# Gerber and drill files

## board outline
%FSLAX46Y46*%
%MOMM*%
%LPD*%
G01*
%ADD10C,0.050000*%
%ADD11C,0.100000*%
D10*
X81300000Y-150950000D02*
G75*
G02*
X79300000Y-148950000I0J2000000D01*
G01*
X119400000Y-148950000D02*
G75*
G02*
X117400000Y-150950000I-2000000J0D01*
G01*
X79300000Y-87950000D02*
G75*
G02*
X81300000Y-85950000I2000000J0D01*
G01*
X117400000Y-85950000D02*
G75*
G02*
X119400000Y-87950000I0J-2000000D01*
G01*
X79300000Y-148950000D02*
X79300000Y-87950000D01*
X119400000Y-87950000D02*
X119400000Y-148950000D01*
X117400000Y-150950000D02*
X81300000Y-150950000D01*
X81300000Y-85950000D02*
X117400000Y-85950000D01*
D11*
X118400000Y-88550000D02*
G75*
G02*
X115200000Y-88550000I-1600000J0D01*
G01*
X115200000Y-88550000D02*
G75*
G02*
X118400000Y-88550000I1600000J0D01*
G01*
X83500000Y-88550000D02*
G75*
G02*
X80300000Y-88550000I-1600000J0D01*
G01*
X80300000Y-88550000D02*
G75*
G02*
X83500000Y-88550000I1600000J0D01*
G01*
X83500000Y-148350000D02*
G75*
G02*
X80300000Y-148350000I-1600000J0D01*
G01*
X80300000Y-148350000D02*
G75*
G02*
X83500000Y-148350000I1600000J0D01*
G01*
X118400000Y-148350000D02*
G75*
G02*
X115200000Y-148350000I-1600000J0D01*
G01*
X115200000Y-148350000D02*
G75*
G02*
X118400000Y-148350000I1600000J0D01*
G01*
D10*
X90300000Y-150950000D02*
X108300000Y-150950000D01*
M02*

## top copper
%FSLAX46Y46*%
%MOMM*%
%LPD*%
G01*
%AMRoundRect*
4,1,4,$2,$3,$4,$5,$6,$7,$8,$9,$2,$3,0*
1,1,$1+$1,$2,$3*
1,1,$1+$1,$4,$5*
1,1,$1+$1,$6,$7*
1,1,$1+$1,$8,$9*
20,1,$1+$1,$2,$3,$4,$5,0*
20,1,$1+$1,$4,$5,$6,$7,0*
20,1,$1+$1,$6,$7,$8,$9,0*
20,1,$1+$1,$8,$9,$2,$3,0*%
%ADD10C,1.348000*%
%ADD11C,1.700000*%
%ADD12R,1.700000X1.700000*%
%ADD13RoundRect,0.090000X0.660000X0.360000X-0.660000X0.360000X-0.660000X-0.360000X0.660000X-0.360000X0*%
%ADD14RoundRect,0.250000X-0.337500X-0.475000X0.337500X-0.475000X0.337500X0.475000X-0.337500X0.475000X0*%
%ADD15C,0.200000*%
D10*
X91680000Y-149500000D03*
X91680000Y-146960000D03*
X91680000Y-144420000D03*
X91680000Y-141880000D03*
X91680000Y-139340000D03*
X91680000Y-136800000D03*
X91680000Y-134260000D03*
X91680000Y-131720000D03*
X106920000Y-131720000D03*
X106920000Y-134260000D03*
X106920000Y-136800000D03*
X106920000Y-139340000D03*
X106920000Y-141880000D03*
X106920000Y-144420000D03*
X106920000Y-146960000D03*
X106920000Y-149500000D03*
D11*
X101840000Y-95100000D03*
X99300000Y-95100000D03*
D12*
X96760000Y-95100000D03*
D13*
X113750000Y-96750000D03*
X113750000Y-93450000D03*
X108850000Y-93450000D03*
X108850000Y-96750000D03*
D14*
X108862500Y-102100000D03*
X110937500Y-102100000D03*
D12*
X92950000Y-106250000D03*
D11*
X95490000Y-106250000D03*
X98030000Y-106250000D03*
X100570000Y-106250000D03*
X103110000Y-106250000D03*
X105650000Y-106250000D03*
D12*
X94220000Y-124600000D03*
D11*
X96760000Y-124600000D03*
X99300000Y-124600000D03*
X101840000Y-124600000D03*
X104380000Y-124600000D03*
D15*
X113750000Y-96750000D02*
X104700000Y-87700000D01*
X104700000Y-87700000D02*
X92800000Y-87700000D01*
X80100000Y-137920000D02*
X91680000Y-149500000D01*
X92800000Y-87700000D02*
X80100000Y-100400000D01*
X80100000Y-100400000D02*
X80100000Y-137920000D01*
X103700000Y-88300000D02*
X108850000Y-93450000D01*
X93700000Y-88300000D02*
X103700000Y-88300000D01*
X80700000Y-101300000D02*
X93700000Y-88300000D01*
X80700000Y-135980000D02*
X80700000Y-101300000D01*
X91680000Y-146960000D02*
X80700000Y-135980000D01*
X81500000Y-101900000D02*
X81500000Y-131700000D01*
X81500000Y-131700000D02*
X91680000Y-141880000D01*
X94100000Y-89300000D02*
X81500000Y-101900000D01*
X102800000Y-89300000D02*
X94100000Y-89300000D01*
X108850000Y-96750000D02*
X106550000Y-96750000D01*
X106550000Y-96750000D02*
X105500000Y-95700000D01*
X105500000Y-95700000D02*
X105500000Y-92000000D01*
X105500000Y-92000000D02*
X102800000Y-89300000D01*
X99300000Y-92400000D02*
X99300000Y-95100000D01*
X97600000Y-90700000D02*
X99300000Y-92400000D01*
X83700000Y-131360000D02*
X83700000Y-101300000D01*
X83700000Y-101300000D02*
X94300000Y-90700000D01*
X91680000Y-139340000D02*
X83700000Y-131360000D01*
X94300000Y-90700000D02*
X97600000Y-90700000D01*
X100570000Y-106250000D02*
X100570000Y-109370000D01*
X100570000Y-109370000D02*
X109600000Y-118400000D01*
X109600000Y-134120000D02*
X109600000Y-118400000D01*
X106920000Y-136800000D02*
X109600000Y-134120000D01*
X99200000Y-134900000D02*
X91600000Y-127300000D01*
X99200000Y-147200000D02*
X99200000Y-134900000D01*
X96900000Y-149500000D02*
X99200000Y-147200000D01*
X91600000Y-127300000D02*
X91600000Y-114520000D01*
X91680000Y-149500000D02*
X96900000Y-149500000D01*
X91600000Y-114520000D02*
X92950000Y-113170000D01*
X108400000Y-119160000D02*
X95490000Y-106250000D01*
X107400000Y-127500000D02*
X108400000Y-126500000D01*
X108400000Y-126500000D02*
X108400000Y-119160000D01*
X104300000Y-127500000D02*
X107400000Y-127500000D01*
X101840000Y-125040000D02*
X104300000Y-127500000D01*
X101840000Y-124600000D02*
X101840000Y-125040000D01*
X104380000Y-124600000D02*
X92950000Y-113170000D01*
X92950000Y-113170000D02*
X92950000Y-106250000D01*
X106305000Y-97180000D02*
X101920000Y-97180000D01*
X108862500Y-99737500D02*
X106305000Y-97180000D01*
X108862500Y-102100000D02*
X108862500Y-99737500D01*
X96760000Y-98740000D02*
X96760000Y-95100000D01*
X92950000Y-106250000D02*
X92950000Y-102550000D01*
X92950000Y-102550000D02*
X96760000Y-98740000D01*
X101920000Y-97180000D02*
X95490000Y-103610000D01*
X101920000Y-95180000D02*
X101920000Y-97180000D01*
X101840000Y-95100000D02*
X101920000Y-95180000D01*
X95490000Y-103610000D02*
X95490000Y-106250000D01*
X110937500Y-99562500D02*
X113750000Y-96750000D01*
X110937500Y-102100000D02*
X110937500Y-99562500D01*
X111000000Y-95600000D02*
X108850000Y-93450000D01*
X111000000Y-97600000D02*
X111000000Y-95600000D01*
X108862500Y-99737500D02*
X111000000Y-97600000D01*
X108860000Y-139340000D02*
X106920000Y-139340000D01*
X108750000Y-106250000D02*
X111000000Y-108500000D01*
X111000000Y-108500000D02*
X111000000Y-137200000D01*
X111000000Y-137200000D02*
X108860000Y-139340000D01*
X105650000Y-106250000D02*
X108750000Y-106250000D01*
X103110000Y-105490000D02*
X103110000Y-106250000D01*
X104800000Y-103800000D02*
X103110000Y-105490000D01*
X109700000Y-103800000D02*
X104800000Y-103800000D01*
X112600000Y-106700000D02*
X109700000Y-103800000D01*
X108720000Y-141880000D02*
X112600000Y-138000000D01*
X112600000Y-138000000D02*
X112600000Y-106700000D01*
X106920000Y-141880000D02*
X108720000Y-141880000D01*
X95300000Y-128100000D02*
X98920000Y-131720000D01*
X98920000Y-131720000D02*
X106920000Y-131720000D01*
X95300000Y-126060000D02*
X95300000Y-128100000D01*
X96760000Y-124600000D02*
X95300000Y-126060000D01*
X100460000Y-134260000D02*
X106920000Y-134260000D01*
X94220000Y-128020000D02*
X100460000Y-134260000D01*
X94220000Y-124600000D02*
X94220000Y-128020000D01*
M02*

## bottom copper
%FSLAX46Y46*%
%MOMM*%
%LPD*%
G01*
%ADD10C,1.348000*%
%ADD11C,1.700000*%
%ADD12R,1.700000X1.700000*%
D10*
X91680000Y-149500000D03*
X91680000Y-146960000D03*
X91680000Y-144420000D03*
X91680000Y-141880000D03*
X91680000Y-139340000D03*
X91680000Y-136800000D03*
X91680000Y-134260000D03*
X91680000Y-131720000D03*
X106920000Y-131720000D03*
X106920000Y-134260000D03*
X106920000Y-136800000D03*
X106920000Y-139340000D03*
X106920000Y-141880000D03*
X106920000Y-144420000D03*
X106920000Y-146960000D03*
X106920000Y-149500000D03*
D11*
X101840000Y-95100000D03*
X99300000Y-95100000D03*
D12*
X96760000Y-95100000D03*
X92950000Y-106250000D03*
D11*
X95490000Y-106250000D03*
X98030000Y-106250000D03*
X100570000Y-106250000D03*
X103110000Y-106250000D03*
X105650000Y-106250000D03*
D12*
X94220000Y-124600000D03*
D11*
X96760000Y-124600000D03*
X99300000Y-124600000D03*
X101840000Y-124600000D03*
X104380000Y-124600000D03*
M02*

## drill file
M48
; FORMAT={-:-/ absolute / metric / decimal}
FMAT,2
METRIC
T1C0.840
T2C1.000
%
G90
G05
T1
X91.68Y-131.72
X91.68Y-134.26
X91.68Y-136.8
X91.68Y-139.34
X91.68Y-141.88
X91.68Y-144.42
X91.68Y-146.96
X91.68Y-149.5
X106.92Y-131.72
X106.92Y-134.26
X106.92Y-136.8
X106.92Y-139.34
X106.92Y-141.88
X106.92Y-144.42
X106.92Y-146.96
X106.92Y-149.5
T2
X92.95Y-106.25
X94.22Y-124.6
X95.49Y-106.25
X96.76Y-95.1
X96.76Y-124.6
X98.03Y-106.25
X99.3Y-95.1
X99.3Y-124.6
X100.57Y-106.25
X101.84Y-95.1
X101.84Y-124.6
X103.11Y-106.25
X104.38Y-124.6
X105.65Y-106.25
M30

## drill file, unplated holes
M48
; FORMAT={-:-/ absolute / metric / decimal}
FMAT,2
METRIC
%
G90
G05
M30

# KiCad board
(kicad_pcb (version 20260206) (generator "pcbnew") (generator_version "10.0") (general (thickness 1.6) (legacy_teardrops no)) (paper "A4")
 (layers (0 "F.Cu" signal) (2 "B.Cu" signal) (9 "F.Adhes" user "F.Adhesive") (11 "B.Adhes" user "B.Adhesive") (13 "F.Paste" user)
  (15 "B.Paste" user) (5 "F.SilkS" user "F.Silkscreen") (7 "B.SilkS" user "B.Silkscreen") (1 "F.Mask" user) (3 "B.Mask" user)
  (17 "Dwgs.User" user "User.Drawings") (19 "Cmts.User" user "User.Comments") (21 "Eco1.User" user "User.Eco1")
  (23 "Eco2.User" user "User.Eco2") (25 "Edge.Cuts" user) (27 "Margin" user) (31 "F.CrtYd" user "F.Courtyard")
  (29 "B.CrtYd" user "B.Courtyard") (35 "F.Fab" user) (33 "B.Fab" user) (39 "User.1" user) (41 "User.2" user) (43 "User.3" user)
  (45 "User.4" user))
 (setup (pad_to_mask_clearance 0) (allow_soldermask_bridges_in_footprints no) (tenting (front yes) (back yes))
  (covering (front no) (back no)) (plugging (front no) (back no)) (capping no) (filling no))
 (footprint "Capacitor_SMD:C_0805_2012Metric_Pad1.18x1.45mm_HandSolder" (layer "F.Cu") (at 109.9 102.1)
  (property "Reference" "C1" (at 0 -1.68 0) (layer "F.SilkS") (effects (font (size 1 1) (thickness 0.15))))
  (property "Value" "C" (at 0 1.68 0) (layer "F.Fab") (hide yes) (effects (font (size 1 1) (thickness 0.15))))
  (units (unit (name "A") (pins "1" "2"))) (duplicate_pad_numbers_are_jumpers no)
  (pad "1" smd roundrect (at -1.0375 0) (size 1.175 1.45) (layers "F.Cu" "F.Mask" "F.Paste") (roundrect_rratio 0.212766) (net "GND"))
  (pad "2" smd roundrect (at 1.0375 0) (size 1.175 1.45) (layers "F.Cu" "F.Mask" "F.Paste") (roundrect_rratio 0.212766) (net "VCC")))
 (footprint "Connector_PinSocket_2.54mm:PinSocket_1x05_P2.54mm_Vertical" (layer "F.Cu") (at 94.22 124.6 90)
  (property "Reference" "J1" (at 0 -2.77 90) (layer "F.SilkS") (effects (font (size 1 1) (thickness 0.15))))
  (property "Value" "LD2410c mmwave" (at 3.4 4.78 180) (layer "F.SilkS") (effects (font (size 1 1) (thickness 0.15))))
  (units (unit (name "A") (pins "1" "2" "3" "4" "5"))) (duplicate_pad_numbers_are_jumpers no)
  (pad "1" thru_hole rect (at 0 0 90) (size 1.7 1.7) (drill 1) (layers "*.Cu" "*.Mask") (remove_unused_layers no) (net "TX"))
  (pad "2" thru_hole circle (at 0 2.54 90) (size 1.7 1.7) (drill 1) (layers "*.Cu" "*.Mask") (remove_unused_layers no) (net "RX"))
  (pad "3" thru_hole circle (at 0 5.08 90) (size 1.7 1.7) (drill 1) (layers "*.Cu" "*.Mask") (remove_unused_layers no) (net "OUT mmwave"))
  (pad "4" thru_hole circle (at 0 7.62 90) (size 1.7 1.7) (drill 1) (layers "*.Cu" "*.Mask") (remove_unused_layers no) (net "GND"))
  (pad "5" thru_hole circle (at 0 10.16 90) (size 1.7 1.7) (drill 1) (layers "*.Cu" "*.Mask") (remove_unused_layers no) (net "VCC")))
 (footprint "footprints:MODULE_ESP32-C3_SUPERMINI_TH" (layer "F.Cu") (at 99.3 139.6 180)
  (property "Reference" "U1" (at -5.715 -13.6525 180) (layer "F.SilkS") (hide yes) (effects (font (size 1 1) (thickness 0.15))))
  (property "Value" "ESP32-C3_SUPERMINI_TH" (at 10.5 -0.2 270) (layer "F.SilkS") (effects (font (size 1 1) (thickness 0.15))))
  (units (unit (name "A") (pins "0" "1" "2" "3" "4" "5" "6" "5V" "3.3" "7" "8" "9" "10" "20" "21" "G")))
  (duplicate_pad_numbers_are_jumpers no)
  (pad "0" thru_hole circle (at 7.62 7.88 180) (size 1.348 1.348) (drill 0.84) (layers "*.Cu" "*.Mask") (remove_unused_layers no)
   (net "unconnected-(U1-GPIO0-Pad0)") (solder_mask_margin 0.102))
  (pad "1" thru_hole circle (at 7.62 5.34 180) (size 1.348 1.348) (drill 0.84) (layers "*.Cu" "*.Mask") (remove_unused_layers no)
   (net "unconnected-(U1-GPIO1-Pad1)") (solder_mask_margin 0.102))
  (pad "2" thru_hole circle (at 7.62 2.8 180) (size 1.348 1.348) (drill 0.84) (layers "*.Cu" "*.Mask") (remove_unused_layers no)
   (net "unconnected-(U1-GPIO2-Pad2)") (solder_mask_margin 0.102))
  (pad "3" thru_hole circle (at 7.62 0.26 180) (size 1.348 1.348) (drill 0.84) (layers "*.Cu" "*.Mask") (remove_unused_layers no)
   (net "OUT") (solder_mask_margin 0.102))
  (pad "3.3" thru_hole circle (at 7.62 -4.82 180) (size 1.348 1.348) (drill 0.84) (layers "*.Cu" "*.Mask") (remove_unused_layers no)
   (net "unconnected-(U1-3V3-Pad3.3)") (solder_mask_margin 0.102))
  (pad "4" thru_hole circle (at 7.62 -2.28 180) (size 1.348 1.348) (drill 0.84) (layers "*.Cu" "*.Mask") (remove_unused_layers no)
   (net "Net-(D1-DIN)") (solder_mask_margin 0.102))
  (pad "5" thru_hole circle (at -7.62 -9.9 180) (size 1.348 1.348) (drill 0.84) (layers "*.Cu" "*.Mask") (remove_unused_layers no)
   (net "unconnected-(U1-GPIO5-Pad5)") (solder_mask_margin 0.102))
  (pad "5V" thru_hole circle (at 7.62 -9.9 180) (size 1.348 1.348) (drill 0.84) (layers "*.Cu" "*.Mask") (remove_unused_layers no)
   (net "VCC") (solder_mask_margin 0.102))
  (pad "6" thru_hole circle (at -7.62 -7.36 180) (size 1.348 1.348) (drill 0.84) (layers "*.Cu" "*.Mask") (remove_unused_layers no)
   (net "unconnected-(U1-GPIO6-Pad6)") (solder_mask_margin 0.102))
  (pad "7" thru_hole circle (at -7.62 -4.82 180) (size 1.348 1.348) (drill 0.84) (layers "*.Cu" "*.Mask") (remove_unused_layers no)
   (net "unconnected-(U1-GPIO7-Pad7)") (solder_mask_margin 0.102))
  (pad "8" thru_hole circle (at -7.62 -2.28 180) (size 1.348 1.348) (drill 0.84) (layers "*.Cu" "*.Mask") (remove_unused_layers no)
   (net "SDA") (solder_mask_margin 0.102))
  (pad "9" thru_hole circle (at -7.62 0.26 180) (size 1.348 1.348) (drill 0.84) (layers "*.Cu" "*.Mask") (remove_unused_layers no)
   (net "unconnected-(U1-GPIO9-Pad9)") (solder_mask_margin 0.102))
  (pad "10" thru_hole circle (at -7.62 2.8 180) (size 1.348 1.348) (drill 0.84) (layers "*.Cu" "*.Mask") (remove_unused_layers no)
   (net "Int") (solder_mask_margin 0.102))
  (pad "20" thru_hole circle (at -7.62 5.34 180) (size 1.348 1.348) (drill 0.84) (layers "*.Cu" "*.Mask") (remove_unused_layers no)
   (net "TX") (solder_mask_margin 0.102))
  (pad "21" thru_hole circle (at -7.62 7.88 180) (size 1.348 1.348) (drill 0.84) (layers "*.Cu" "*.Mask") (remove_unused_layers no)
   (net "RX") (solder_mask_margin 0.102))
  (pad "G" thru_hole circle (at 7.62 -7.36 180) (size 1.348 1.348) (drill 0.84) (layers "*.Cu" "*.Mask") (remove_unused_layers no)
   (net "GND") (solder_mask_margin 0.102)))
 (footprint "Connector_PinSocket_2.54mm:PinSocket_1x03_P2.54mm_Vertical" (layer "F.Cu") (at 96.76 95.1 90)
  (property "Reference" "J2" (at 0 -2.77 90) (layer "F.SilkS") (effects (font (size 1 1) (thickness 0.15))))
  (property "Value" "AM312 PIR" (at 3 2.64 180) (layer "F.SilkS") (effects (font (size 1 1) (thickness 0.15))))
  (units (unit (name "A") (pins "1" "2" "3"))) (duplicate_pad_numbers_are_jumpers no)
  (pad "1" thru_hole rect (at 0 0 90) (size 1.7 1.7) (drill 1) (layers "*.Cu" "*.Mask") (remove_unused_layers no) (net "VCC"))
  (pad "2" thru_hole circle (at 0 2.54 90) (size 1.7 1.7) (drill 1) (layers "*.Cu" "*.Mask") (remove_unused_layers no) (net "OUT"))
  (pad "3" thru_hole circle (at 0 5.08 90) (size 1.7 1.7) (drill 1) (layers "*.Cu" "*.Mask") (remove_unused_layers no) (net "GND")))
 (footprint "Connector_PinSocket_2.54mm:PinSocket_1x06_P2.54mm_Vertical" (layer "F.Cu") (at 92.95 106.25 90)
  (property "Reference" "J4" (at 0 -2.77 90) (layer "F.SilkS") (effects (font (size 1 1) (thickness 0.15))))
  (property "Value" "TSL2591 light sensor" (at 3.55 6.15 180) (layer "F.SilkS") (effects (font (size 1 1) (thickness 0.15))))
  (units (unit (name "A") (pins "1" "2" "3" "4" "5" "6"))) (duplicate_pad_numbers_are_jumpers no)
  (pad "1" thru_hole rect (at 0 0 90) (size 1.7 1.7) (drill 1) (layers "*.Cu" "*.Mask") (remove_unused_layers no) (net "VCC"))
  (pad "2" thru_hole circle (at 0 2.54 90) (size 1.7 1.7) (drill 1) (layers "*.Cu" "*.Mask") (remove_unused_layers no) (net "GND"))
  (pad "3" thru_hole circle (at 0 5.08 90) (size 1.7 1.7) (drill 1) (layers "*.Cu" "*.Mask") (remove_unused_layers no) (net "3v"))
  (pad "4" thru_hole circle (at 0 7.62 90) (size 1.7 1.7) (drill 1) (layers "*.Cu" "*.Mask") (remove_unused_layers no) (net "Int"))
  (pad "5" thru_hole circle (at 0 10.16 90) (size 1.7 1.7) (drill 1) (layers "*.Cu" "*.Mask") (remove_unused_layers no) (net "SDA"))
  (pad "6" thru_hole circle (at 0 12.7 90) (size 1.7 1.7) (drill 1) (layers "*.Cu" "*.Mask") (remove_unused_layers no) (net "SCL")))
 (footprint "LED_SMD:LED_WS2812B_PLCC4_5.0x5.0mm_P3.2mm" (layer "F.Cu") (at 111.3 95.1 180)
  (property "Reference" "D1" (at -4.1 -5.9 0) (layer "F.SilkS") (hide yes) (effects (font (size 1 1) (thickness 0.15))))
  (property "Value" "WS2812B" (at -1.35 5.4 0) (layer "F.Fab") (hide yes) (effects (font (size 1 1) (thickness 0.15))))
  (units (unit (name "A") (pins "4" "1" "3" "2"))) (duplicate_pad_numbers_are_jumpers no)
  (pad "1" smd roundrect (at -2.45 -1.65 180) (size 1.5 0.9) (layers "F.Cu" "F.Mask" "F.Paste") (roundrect_rratio 0.1) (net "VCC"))
  (pad "2" smd roundrect (at -2.45 1.65 180) (size 1.5 0.9) (layers "F.Cu" "F.Mask" "F.Paste") (roundrect_rratio 0.1)
   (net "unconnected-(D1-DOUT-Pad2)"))
  (pad "3" smd roundrect (at 2.45 1.65 180) (size 1.5 0.9) (layers "F.Cu" "F.Mask" "F.Paste") (roundrect_rratio 0.1) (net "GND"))
  (pad "4" smd roundrect (at 2.45 -1.65 180) (size 1.5 0.9) (layers "F.Cu" "F.Mask" "F.Paste") (roundrect_rratio 0.1) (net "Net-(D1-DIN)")))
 (gr_arc (start 79.3 87.95) (mid 79.885786 86.535786) (end 81.3 85.95) (stroke (width 0.05) (type default)) (layer "Edge.Cuts"))
 (gr_line (start 79.3 148.95) (end 79.3 87.95) (stroke (width 0.05) (type default)) (layer "Edge.Cuts"))
 (gr_line (start 81.3 85.95) (end 117.4 85.95) (stroke (width 0.05) (type default)) (layer "Edge.Cuts"))
 (gr_arc (start 81.3 150.95) (mid 79.885786 150.364214) (end 79.3 148.95) (stroke (width 0.05) (type default)) (layer "Edge.Cuts"))
 (gr_circle (center 81.9 88.55) (end 80.3 88.55) (stroke (width 0.1) (type solid)) (fill no) (layer "Edge.Cuts"))
 (gr_circle (center 81.9 148.35) (end 81.9 149.95) (stroke (width 0.1) (type solid)) (fill no) (layer "Edge.Cuts"))
 (gr_line (start 90.3 150.95) (end 108.3 150.95) (stroke (width 0.05) (type default)) (layer "Edge.Cuts"))
 (gr_circle (center 116.8 88.55) (end 116.8 86.95) (stroke (width 0.1) (type solid)) (fill no) (layer "Edge.Cuts"))
 (gr_circle (center 116.8 148.35) (end 118.4 148.35) (stroke (width 0.1) (type solid)) (fill no) (layer "Edge.Cuts"))
 (gr_arc (start 117.4 85.95) (mid 118.814214 86.535786) (end 119.4 87.95) (stroke (width 0.05) (type default)) (layer "Edge.Cuts"))
 (gr_line (start 117.4 150.95) (end 81.3 150.95) (stroke (width 0.05) (type default)) (layer "Edge.Cuts"))
 (gr_line (start 119.4 87.95) (end 119.4 148.95) (stroke (width 0.05) (type default)) (layer "Edge.Cuts"))
 (gr_arc (start 119.4 148.95) (mid 118.814214 150.364214) (end 117.4 150.95) (stroke (width 0.05) (type default)) (layer "Edge.Cuts"))
 (segment (start 106.305 97.18) (end 101.92 97.18) (width 0.2) (layer "F.Cu") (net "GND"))
 (segment (start 108.8625 99.7375) (end 111 97.6) (width 0.2) (layer "F.Cu") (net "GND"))
 (segment (start 108.8625 102.1) (end 108.8625 99.7375) (width 0.2) (layer "F.Cu") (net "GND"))
 (segment (start 95.49 103.61) (end 95.49 106.25) (width 0.2) (layer "F.Cu") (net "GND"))
 (segment (start 101.84 124.6) (end 101.84 125.04) (width 0.2) (layer "F.Cu") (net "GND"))
 (segment (start 108.4 126.5) (end 108.4 119.16) (width 0.2) (layer "F.Cu") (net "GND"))
 (segment (start 93.7 88.3) (end 103.7 88.3) (width 0.2) (layer "F.Cu") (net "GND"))
 (segment (start 101.84 125.04) (end 104.3 127.5) (width 0.2) (layer "F.Cu") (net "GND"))
 (segment (start 80.7 101.3) (end 93.7 88.3) (width 0.2) (layer "F.Cu") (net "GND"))
 (segment (start 111 95.6) (end 108.85 93.45) (width 0.2) (layer "F.Cu") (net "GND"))
 (segment (start 104.3 127.5) (end 107.4 127.5) (width 0.2) (layer "F.Cu") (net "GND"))
 (segment (start 108.4 119.16) (end 95.49 106.25) (width 0.2) (layer "F.Cu") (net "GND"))
 (segment (start 101.92 97.18) (end 95.49 103.61) (width 0.2) (layer "F.Cu") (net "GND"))
 (segment (start 108.8625 99.7375) (end 106.305 97.18) (width 0.2) (layer "F.Cu") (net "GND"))
 (segment (start 111 97.6) (end 111 95.6) (width 0.2) (layer "F.Cu") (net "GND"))
 (segment (start 101.92 95.18) (end 101.92 97.18) (width 0.2) (layer "F.Cu") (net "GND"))
 (segment (start 80.7 135.98) (end 80.7 101.3) (width 0.2) (layer "F.Cu") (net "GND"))
 (segment (start 101.84 95.1) (end 101.92 95.18) (width 0.2) (layer "F.Cu") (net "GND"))
 (segment (start 107.4 127.5) (end 108.4 126.5) (width 0.2) (layer "F.Cu") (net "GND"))
 (segment (start 91.68 146.96) (end 80.7 135.98) (width 0.2) (layer "F.Cu") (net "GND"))
 (segment (start 103.7 88.3) (end 108.85 93.45) (width 0.2) (layer "F.Cu") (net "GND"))
 (segment (start 91.68 149.5) (end 96.9 149.5) (width 0.2) (layer "F.Cu") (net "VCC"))
 (segment (start 99.2 134.9) (end 91.6 127.3) (width 0.2) (layer "F.Cu") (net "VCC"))
 (segment (start 92.8 87.7) (end 80.1 100.4) (width 0.2) (layer "F.Cu") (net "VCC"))
 (segment (start 96.9 149.5) (end 99.2 147.2) (width 0.2) (layer "F.Cu") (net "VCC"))
 (segment (start 110.9375 99.5625) (end 113.75 96.75) (width 0.2) (layer "F.Cu") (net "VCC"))
 (segment (start 99.2 147.2) (end 99.2 134.9) (width 0.2) (layer "F.Cu") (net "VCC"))
 (segment (start 80.1 100.4) (end 80.1 137.92) (width 0.2) (layer "F.Cu") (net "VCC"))
 (segment (start 91.6 114.52) (end 92.95 113.17) (width 0.2) (layer "F.Cu") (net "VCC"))
 (segment (start 92.95 106.25) (end 92.95 102.55) (width 0.2) (layer "F.Cu") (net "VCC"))
 (segment (start 96.76 98.74) (end 96.76 95.1) (width 0.2) (layer "F.Cu") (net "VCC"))
 (segment (start 104.38 124.6) (end 92.95 113.17) (width 0.2) (layer "F.Cu") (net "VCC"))
 (segment (start 80.1 137.92) (end 91.68 149.5) (width 0.2) (layer "F.Cu") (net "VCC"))
 (segment (start 110.9375 102.1) (end 110.9375 99.5625) (width 0.2) (layer "F.Cu") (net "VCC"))
 (segment (start 91.6 127.3) (end 91.6 114.52) (width 0.2) (layer "F.Cu") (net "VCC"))
 (segment (start 92.95 113.17) (end 92.95 106.25) (width 0.2) (layer "F.Cu") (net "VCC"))
 (segment (start 104.7 87.7) (end 92.8 87.7) (width 0.2) (layer "F.Cu") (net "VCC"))
 (segment (start 92.95 102.55) (end 96.76 98.74) (width 0.2) (layer "F.Cu") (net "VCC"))
 (segment (start 113.75 96.75) (end 104.7 87.7) (width 0.2) (layer "F.Cu") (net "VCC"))
 (segment (start 81.5 101.9) (end 81.5 131.7) (width 0.2) (layer "F.Cu") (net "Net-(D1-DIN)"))
 (segment (start 105.5 95.7) (end 105.5 92) (width 0.2) (layer "F.Cu") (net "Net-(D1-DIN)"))
 (segment (start 94.1 89.3) (end 81.5 101.9) (width 0.2) (layer "F.Cu") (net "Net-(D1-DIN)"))
 (segment (start 106.55 96.75) (end 105.5 95.7) (width 0.2) (layer "F.Cu") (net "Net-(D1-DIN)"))
 (segment (start 108.85 96.75) (end 106.55 96.75) (width 0.2) (layer "F.Cu") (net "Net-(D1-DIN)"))
 (segment (start 105.5 92) (end 102.8 89.3) (width 0.2) (layer "F.Cu") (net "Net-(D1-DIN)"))
 (segment (start 102.8 89.3) (end 94.1 89.3) (width 0.2) (layer "F.Cu") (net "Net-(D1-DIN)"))
 (segment (start 81.5 131.7) (end 91.68 141.88) (width 0.2) (layer "F.Cu") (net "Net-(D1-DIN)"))
 (segment (start 94.22 128.02) (end 100.46 134.26) (width 0.2) (layer "F.Cu") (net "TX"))
 (segment (start 100.46 134.26) (end 106.92 134.26) (width 0.2) (layer "F.Cu") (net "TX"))
 (segment (start 94.22 124.6) (end 94.22 128.02) (width 0.2) (layer "F.Cu") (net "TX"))
 (segment (start 83.7 131.36) (end 83.7 101.3) (width 0.2) (layer "F.Cu") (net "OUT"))
 (segment (start 99.3 92.4) (end 99.3 95.1) (width 0.2) (layer "F.Cu") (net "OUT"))
 (segment (start 83.7 101.3) (end 94.3 90.7) (width 0.2) (layer "F.Cu") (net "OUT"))
 (segment (start 97.6 90.7) (end 99.3 92.4) (width 0.2) (layer "F.Cu") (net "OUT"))
 (segment (start 91.68 139.34) (end 83.7 131.36) (width 0.2) (layer "F.Cu") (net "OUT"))
 (segment (start 94.3 90.7) (end 97.6 90.7) (width 0.2) (layer "F.Cu") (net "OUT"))
 (segment (start 96.76 124.6) (end 95.3 126.06) (width 0.2) (layer "F.Cu") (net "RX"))
 (segment (start 98.92 131.72) (end 106.92 131.72) (width 0.2) (layer "F.Cu") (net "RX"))
 (segment (start 95.3 126.06) (end 95.3 128.1) (width 0.2) (layer "F.Cu") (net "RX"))
 (segment (start 95.3 128.1) (end 98.92 131.72) (width 0.2) (layer "F.Cu") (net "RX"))
 (segment (start 106.92 141.88) (end 108.72 141.88) (width 0.2) (layer "F.Cu") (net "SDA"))
 (segment (start 104.8 103.8) (end 103.11 105.49) (width 0.2) (layer "F.Cu") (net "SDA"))
 (segment (start 112.6 106.7) (end 109.7 103.8) (width 0.2) (layer "F.Cu") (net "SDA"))
 (segment (start 109.7 103.8) (end 104.8 103.8) (width 0.2) (layer "F.Cu") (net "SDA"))
 (segment (start 108.72 141.88) (end 112.6 138) (width 0.2) (layer "F.Cu") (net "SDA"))
 (segment (start 112.6 138) (end 112.6 106.7) (width 0.2) (layer "F.Cu") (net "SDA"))
 (segment (start 103.11 105.49) (end 103.11 106.25) (width 0.2) (layer "F.Cu") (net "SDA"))
 (segment (start 108.75 106.25) (end 111 108.5) (width 0.2) (layer "F.Cu") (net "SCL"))
 (segment (start 105.65 106.25) (end 108.75 106.25) (width 0.2) (layer "F.Cu") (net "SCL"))
 (segment (start 108.86 139.34) (end 106.92 139.34) (width 0.2) (layer "F.Cu") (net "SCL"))
 (segment (start 111 108.5) (end 111 137.2) (width 0.2) (layer "F.Cu") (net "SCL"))
 (segment (start 111 137.2) (end 108.86 139.34) (width 0.2) (layer "F.Cu") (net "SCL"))
 (segment (start 100.57 109.37) (end 109.6 118.4) (width 0.2) (layer "F.Cu") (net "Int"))
 (segment (start 100.57 106.25) (end 100.57 109.37) (width 0.2) (layer "F.Cu") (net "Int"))
 (segment (start 109.6 134.12) (end 109.6 118.4) (width 0.2) (layer "F.Cu") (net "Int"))
 (segment (start 106.92 136.8) (end 109.6 134.12) (width 0.2) (layer "F.Cu") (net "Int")))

